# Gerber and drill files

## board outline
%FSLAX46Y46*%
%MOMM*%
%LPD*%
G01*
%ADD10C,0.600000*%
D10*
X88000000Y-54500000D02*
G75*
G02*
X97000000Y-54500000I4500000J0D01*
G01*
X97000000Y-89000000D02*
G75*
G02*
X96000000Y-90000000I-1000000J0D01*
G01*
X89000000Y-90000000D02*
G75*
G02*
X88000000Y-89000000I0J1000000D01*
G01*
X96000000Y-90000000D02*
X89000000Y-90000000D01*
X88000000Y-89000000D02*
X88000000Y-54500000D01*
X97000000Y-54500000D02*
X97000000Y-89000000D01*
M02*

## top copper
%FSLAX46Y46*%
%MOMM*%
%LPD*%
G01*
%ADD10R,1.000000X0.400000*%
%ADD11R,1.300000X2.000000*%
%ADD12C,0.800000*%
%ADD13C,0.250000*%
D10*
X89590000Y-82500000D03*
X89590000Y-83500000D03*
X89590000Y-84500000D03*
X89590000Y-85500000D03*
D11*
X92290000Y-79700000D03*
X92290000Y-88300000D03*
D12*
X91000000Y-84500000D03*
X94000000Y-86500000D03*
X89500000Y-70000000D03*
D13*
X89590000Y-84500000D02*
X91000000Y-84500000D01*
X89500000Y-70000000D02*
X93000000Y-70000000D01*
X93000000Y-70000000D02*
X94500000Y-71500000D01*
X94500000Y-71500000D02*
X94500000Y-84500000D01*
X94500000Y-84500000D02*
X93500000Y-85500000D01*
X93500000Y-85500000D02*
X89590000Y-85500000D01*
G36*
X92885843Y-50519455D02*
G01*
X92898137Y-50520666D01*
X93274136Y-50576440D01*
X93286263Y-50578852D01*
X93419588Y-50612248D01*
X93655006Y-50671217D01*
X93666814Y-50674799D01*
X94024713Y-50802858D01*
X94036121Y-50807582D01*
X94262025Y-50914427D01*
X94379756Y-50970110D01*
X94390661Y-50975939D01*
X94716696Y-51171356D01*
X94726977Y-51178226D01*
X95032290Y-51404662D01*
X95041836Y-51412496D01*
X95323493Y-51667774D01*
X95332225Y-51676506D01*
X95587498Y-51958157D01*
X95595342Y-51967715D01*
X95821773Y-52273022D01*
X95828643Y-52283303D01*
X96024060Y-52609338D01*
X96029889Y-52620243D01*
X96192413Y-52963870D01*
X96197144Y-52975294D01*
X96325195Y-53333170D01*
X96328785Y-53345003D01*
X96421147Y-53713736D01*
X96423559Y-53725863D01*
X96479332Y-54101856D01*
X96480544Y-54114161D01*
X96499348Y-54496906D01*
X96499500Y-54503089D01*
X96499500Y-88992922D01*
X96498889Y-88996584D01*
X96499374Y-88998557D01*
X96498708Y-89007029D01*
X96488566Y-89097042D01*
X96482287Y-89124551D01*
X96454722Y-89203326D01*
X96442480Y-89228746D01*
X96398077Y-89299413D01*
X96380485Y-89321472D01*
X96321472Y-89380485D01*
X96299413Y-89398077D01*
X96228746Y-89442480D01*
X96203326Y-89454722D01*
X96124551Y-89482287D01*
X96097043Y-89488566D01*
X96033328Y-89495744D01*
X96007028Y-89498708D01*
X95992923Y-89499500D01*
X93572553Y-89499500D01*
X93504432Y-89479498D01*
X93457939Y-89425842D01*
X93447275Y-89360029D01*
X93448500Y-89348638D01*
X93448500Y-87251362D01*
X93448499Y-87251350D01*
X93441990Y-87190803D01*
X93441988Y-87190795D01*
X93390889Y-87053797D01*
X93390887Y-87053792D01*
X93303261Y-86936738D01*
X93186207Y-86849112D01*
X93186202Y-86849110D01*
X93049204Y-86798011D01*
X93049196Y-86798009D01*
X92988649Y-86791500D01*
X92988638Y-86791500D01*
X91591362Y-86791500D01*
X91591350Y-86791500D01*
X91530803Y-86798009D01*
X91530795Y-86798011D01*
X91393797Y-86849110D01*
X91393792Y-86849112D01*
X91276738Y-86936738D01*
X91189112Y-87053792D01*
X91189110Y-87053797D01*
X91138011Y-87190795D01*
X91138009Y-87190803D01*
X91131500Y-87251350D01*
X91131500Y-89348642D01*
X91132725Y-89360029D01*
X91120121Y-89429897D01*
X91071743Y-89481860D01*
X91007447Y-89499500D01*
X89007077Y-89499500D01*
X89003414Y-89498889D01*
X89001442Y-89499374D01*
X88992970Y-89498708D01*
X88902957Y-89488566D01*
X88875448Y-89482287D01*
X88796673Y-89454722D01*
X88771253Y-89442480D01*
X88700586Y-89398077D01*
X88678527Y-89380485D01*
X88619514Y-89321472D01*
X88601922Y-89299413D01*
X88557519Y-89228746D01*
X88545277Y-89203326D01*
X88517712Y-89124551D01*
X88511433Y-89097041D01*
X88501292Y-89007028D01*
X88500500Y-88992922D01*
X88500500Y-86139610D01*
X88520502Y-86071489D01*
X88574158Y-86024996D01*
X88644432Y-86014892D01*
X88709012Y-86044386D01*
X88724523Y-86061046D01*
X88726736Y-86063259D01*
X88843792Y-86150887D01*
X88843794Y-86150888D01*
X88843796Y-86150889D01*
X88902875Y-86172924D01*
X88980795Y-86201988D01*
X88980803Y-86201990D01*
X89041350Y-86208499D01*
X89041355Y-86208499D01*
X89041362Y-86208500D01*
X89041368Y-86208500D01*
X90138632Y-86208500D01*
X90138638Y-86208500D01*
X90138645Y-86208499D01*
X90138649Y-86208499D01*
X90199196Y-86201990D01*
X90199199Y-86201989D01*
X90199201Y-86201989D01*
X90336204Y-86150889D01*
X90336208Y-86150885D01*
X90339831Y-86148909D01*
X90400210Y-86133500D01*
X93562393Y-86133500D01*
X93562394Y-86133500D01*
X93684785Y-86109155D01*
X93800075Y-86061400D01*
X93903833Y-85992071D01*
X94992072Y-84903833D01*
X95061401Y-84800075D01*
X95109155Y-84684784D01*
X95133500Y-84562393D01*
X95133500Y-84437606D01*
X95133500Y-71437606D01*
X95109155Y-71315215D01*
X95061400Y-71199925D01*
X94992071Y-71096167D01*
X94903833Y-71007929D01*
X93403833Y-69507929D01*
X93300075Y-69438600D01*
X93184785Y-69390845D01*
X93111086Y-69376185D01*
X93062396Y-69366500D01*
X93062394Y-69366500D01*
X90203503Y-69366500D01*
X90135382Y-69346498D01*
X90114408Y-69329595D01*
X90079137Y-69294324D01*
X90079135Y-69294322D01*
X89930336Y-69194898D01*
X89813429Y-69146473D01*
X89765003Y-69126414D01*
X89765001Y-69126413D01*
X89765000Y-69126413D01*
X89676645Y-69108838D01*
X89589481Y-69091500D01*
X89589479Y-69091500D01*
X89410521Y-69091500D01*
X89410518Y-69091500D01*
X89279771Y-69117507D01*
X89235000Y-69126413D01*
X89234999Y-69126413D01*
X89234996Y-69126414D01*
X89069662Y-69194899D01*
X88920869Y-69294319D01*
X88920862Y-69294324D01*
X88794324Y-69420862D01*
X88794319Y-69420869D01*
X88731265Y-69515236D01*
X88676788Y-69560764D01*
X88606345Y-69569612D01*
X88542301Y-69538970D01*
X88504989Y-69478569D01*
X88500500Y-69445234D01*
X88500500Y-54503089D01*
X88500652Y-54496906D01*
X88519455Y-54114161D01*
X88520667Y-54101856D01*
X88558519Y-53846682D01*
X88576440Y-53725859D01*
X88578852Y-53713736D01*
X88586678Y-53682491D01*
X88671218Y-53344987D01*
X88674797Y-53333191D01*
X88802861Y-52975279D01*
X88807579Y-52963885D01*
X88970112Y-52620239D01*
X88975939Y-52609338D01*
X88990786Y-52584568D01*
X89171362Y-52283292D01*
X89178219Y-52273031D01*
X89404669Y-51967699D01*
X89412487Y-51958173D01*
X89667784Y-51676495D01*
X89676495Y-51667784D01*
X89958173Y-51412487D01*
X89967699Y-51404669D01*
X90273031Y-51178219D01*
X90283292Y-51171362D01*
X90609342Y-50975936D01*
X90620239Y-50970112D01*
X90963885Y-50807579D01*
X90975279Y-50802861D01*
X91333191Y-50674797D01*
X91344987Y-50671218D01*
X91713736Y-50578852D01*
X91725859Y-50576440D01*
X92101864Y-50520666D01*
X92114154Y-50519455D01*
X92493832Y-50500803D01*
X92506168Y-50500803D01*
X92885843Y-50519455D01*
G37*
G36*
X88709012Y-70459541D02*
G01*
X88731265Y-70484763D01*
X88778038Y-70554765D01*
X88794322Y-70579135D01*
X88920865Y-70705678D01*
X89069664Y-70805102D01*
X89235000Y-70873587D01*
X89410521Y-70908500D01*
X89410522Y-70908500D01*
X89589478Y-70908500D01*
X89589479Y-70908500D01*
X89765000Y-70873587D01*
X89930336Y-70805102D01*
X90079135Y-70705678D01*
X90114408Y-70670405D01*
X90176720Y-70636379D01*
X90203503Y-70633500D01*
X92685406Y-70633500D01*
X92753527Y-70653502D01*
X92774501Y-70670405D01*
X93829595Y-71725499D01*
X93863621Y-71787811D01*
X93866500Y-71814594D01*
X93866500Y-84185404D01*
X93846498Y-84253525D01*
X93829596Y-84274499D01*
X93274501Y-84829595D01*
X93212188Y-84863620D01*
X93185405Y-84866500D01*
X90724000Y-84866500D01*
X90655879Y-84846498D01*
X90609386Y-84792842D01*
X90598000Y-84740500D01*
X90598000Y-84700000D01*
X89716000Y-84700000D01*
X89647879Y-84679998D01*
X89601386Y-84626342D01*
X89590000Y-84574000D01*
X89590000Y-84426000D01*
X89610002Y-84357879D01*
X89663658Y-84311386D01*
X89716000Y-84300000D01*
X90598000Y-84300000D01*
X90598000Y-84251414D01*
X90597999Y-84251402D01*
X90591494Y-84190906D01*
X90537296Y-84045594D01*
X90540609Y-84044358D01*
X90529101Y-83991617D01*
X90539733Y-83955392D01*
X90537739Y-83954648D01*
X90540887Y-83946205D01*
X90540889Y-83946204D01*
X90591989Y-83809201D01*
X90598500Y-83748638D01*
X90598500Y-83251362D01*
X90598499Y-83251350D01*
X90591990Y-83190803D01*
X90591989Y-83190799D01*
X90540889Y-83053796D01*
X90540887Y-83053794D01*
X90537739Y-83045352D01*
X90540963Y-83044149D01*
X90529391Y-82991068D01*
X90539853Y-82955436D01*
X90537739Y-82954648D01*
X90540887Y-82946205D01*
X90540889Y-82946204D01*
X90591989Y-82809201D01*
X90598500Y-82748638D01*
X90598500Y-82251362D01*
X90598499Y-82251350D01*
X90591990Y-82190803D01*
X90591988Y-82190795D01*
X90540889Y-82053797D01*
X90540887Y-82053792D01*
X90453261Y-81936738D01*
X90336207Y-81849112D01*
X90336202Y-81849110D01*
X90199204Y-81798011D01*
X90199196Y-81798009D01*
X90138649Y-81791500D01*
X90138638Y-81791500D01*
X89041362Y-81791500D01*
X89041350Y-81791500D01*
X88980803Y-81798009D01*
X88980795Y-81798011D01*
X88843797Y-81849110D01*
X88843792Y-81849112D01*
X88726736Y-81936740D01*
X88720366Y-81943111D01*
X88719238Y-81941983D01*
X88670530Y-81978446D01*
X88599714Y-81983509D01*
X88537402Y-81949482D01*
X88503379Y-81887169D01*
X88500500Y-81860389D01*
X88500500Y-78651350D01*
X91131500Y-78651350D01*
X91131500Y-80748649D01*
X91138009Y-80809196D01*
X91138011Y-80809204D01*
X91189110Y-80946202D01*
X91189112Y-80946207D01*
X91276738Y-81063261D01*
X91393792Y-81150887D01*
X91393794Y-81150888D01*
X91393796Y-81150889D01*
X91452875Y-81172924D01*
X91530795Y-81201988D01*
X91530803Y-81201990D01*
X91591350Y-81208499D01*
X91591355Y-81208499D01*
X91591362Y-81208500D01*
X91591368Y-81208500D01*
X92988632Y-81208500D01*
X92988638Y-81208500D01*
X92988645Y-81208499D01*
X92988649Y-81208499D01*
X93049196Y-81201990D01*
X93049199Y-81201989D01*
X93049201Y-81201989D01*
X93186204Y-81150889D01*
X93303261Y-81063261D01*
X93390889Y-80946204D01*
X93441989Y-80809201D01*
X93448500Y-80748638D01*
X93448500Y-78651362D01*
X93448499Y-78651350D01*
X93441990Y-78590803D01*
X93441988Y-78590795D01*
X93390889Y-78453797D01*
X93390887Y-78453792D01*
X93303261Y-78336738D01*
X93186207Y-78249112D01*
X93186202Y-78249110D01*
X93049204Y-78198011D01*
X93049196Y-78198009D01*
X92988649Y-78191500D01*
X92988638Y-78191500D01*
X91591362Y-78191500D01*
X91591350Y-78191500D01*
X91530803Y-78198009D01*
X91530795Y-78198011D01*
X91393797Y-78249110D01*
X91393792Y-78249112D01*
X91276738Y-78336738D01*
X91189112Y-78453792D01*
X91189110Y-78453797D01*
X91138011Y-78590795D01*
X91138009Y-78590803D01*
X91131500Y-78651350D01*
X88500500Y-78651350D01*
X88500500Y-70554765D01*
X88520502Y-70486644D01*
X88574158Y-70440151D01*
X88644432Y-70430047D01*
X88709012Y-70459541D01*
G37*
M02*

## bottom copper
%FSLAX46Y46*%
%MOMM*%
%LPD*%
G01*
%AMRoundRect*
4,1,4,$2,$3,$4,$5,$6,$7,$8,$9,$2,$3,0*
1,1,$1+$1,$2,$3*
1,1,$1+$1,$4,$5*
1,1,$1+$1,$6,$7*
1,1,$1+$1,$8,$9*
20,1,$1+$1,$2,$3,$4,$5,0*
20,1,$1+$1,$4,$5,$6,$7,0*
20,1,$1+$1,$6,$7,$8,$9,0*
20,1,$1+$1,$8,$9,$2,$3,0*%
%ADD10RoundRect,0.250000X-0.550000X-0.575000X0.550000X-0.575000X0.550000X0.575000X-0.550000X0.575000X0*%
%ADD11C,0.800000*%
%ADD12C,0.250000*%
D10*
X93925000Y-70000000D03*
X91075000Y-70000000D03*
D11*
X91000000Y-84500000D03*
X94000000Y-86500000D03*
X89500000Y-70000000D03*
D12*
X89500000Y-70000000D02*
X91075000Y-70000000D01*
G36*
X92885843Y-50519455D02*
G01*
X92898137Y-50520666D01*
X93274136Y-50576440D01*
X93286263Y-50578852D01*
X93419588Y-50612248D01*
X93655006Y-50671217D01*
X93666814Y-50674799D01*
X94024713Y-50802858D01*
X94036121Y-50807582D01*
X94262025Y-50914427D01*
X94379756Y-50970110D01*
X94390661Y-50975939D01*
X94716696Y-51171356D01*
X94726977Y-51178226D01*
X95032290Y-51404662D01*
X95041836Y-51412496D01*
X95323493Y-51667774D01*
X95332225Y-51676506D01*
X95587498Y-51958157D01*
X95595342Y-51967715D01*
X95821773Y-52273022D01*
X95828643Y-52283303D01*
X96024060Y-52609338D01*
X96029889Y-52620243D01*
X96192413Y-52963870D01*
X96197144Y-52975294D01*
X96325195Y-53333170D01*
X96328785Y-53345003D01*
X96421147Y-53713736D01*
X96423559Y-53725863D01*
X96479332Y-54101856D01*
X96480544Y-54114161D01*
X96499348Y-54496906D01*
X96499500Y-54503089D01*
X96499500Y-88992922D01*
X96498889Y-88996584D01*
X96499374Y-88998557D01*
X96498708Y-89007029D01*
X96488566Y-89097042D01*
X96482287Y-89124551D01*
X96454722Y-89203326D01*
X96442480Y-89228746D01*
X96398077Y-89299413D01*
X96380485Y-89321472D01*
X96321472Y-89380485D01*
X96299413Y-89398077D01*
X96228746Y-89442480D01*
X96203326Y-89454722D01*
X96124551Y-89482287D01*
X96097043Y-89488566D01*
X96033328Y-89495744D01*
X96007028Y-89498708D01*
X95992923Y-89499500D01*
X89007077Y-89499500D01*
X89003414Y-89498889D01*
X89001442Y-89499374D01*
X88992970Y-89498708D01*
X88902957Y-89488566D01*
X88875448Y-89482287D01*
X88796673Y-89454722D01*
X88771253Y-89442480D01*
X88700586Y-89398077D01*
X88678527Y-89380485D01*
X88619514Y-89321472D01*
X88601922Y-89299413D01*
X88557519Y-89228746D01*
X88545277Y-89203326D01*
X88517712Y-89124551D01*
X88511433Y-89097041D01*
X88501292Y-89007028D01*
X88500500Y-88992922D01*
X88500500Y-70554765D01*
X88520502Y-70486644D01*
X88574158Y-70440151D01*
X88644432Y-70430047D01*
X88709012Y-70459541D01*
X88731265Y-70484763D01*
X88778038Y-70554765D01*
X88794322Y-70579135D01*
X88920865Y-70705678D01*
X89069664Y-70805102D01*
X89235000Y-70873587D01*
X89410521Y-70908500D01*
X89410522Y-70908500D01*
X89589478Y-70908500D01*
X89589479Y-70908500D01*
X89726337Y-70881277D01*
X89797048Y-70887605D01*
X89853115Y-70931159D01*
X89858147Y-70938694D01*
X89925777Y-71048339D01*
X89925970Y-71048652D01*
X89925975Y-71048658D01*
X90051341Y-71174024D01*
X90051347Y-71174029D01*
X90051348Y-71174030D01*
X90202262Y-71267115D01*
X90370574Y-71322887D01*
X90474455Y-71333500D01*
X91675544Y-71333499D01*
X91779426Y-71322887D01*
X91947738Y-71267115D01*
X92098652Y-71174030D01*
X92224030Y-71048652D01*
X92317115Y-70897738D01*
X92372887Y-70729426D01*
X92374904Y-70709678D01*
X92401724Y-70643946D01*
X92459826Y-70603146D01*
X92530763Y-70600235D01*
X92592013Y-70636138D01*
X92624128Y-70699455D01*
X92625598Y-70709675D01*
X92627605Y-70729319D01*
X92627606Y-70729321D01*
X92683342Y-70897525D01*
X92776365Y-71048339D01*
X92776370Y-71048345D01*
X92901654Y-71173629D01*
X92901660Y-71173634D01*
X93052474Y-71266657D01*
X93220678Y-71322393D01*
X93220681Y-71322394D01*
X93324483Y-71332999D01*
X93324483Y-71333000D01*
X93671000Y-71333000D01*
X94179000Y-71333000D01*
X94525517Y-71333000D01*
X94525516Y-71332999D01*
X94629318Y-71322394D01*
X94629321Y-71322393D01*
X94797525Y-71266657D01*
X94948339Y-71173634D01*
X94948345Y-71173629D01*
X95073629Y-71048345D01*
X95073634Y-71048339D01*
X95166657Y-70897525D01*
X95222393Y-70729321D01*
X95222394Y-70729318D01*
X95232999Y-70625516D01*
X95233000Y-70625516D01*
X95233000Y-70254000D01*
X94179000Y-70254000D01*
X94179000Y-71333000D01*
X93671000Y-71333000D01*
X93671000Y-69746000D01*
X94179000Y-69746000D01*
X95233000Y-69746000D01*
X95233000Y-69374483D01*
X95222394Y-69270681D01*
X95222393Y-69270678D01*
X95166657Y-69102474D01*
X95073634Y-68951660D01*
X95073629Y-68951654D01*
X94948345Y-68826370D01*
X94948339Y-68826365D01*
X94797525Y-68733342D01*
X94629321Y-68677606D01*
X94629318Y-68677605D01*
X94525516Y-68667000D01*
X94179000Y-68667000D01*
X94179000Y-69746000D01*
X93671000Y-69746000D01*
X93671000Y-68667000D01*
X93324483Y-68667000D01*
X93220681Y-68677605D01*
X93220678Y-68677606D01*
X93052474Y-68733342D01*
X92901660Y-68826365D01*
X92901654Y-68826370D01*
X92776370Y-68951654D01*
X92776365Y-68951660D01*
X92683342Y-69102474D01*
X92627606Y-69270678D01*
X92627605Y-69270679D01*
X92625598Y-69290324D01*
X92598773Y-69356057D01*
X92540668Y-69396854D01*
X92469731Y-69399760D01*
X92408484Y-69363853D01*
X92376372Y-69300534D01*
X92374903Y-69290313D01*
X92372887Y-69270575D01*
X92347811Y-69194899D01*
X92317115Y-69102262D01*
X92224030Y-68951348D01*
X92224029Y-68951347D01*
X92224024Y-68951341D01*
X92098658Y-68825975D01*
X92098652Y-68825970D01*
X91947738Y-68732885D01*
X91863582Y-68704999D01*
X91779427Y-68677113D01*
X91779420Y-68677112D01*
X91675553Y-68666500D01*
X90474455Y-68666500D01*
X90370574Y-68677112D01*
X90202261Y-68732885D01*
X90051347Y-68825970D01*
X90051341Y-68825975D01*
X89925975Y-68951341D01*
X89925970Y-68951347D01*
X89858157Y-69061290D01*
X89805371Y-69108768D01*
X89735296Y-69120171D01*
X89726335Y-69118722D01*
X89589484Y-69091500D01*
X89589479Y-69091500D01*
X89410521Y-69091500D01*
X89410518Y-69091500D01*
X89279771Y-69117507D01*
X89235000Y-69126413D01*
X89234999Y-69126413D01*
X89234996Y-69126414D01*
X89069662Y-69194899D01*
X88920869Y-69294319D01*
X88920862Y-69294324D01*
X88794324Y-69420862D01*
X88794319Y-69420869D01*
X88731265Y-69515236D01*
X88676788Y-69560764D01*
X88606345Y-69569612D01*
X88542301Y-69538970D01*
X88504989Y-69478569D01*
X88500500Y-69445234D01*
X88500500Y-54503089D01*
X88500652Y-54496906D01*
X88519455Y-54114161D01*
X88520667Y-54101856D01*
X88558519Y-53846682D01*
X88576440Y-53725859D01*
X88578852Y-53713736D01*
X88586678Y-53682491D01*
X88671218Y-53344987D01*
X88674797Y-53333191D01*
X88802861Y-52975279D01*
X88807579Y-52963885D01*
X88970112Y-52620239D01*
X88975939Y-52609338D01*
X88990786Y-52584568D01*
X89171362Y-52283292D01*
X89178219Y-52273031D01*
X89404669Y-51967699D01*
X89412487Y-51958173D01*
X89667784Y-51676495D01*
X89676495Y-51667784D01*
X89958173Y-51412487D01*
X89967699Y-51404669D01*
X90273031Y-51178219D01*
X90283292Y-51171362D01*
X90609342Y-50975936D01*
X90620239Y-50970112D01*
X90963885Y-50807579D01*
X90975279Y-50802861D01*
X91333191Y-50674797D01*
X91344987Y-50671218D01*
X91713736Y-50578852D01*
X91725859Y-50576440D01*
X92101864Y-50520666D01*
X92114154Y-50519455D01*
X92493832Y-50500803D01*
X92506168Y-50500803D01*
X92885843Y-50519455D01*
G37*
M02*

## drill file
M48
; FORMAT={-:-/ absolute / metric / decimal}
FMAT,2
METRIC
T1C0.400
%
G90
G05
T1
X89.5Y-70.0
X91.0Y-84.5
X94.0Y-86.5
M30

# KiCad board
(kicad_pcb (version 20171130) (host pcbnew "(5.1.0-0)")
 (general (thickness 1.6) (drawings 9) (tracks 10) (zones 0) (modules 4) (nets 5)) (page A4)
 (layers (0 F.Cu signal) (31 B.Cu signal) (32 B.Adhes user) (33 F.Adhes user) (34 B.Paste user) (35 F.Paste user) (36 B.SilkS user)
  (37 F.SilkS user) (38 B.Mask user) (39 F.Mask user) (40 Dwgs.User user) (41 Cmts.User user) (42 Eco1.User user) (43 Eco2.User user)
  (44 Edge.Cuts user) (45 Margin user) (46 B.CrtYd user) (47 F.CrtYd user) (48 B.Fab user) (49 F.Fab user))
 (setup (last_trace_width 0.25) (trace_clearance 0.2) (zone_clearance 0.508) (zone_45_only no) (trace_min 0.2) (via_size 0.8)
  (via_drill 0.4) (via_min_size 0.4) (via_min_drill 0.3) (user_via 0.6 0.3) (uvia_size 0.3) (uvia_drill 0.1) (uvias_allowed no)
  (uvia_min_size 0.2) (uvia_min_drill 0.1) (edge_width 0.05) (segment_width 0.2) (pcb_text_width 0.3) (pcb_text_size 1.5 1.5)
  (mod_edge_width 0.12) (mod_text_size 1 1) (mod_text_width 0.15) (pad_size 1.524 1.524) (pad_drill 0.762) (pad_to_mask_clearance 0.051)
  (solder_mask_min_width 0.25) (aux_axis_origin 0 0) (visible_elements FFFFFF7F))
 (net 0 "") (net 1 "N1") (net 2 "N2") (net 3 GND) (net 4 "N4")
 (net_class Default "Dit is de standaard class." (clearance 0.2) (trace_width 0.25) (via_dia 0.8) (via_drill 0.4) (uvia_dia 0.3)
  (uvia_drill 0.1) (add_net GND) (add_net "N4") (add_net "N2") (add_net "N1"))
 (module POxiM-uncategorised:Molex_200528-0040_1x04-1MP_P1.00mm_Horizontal (layer F.Cu) (at 90.5 84 90)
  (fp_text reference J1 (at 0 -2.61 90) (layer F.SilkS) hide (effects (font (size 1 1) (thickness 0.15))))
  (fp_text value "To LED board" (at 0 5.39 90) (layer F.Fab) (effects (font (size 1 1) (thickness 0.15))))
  (pad 4 smd rect (at 1.5 -0.91 90) (size 0.4 1) (layers F.Cu F.Paste F.Mask) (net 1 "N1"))
  (pad 3 smd rect (at 0.5 -0.91 90) (size 0.4 1) (layers F.Cu F.Paste F.Mask) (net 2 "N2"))
  (pad 2 smd rect (at -0.5 -0.91 90) (size 0.4 1) (layers F.Cu F.Paste F.Mask) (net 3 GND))
  (pad 1 smd rect (at -1.5 -0.91 90) (size 0.4 1) (layers F.Cu F.Paste F.Mask) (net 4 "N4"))
  (pad MP smd rect (at 4.3 1.79 90) (size 2 1.3) (layers F.Cu F.Paste F.Mask))
  (pad MP smd rect (at -4.3 1.79 90) (size 2 1.3) (layers F.Cu F.Paste F.Mask)))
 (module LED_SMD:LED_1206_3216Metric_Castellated (layer B.Cu) (at 92.5 70)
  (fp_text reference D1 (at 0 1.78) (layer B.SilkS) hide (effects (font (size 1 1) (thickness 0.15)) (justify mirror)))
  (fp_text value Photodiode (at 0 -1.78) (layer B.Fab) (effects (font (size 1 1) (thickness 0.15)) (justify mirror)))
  (pad 2 smd roundrect (at 1.425 0) (size 1.6 1.65) (layers B.Cu B.Paste B.Mask) (roundrect_rratio 0.15625) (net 3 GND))
  (pad 1 smd roundrect (at -1.425 0) (size 1.6 1.65) (layers B.Cu B.Paste B.Mask) (roundrect_rratio 0.15625) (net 4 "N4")))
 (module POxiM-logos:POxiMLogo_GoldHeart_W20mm (layer F.Cu) (at 91.75 67.5 90)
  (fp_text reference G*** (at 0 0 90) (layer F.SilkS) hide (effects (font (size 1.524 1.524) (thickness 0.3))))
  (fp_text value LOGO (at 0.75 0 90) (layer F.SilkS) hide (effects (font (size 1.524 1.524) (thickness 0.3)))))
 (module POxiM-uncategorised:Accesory (layer F.Cu) (at 40 145)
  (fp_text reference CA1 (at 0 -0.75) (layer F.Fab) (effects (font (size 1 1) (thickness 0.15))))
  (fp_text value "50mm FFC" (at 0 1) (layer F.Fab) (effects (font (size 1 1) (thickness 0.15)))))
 (gr_arc (start 92.5 54.5) (end 97 54.5) (angle -180) (layer Edge.Cuts) (width 0.6))
 (gr_arc (start 96 89) (end 96 90) (angle -90) (layer Edge.Cuts) (width 0.6))
 (gr_arc (start 89 89) (end 88 89) (angle -90) (layer Edge.Cuts) (width 0.6))
 (gr_line (start 96 90) (end 89 90) (layer Edge.Cuts) (width 0.6))
 (gr_line (start 88 89) (end 88 54.5) (layer Edge.Cuts) (width 0.6))
 (gr_line (start 97 54.5) (end 97 89) (layer Edge.Cuts) (width 0.6))
 (via (at 91 84.5) (size 0.8) (drill 0.4) (layers F.Cu B.Cu) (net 3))
 (via (at 94 86.5) (size 0.8) (drill 0.4) (layers F.Cu B.Cu) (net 3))
 (segment (start 89.59 84.5) (end 91 84.5) (width 0.25) (layer F.Cu) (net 3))
 (via (at 89.5 70) (size 0.8) (drill 0.4) (layers F.Cu B.Cu) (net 4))
 (segment (start 89.5 70) (end 93 70) (width 0.25) (layer F.Cu) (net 4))
 (segment (start 93 70) (end 94.5 71.5) (width 0.25) (layer F.Cu) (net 4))
 (segment (start 94.5 71.5) (end 94.5 84.5) (width 0.25) (layer F.Cu) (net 4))
 (segment (start 94.5 84.5) (end 93.5 85.5) (width 0.25) (layer F.Cu) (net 4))
 (segment (start 93.5 85.5) (end 89.59 85.5) (width 0.25) (layer F.Cu) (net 4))
 (segment (start 89.5 70) (end 91.075 70) (width 0.25) (layer B.Cu) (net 4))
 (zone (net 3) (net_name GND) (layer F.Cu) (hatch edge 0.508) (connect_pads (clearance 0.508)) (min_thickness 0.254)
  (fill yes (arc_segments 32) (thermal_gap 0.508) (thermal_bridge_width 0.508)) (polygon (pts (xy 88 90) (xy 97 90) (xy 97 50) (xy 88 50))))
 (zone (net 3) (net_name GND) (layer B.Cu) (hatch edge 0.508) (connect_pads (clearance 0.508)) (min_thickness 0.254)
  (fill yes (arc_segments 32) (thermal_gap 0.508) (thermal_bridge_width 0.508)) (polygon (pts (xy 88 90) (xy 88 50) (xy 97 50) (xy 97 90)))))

